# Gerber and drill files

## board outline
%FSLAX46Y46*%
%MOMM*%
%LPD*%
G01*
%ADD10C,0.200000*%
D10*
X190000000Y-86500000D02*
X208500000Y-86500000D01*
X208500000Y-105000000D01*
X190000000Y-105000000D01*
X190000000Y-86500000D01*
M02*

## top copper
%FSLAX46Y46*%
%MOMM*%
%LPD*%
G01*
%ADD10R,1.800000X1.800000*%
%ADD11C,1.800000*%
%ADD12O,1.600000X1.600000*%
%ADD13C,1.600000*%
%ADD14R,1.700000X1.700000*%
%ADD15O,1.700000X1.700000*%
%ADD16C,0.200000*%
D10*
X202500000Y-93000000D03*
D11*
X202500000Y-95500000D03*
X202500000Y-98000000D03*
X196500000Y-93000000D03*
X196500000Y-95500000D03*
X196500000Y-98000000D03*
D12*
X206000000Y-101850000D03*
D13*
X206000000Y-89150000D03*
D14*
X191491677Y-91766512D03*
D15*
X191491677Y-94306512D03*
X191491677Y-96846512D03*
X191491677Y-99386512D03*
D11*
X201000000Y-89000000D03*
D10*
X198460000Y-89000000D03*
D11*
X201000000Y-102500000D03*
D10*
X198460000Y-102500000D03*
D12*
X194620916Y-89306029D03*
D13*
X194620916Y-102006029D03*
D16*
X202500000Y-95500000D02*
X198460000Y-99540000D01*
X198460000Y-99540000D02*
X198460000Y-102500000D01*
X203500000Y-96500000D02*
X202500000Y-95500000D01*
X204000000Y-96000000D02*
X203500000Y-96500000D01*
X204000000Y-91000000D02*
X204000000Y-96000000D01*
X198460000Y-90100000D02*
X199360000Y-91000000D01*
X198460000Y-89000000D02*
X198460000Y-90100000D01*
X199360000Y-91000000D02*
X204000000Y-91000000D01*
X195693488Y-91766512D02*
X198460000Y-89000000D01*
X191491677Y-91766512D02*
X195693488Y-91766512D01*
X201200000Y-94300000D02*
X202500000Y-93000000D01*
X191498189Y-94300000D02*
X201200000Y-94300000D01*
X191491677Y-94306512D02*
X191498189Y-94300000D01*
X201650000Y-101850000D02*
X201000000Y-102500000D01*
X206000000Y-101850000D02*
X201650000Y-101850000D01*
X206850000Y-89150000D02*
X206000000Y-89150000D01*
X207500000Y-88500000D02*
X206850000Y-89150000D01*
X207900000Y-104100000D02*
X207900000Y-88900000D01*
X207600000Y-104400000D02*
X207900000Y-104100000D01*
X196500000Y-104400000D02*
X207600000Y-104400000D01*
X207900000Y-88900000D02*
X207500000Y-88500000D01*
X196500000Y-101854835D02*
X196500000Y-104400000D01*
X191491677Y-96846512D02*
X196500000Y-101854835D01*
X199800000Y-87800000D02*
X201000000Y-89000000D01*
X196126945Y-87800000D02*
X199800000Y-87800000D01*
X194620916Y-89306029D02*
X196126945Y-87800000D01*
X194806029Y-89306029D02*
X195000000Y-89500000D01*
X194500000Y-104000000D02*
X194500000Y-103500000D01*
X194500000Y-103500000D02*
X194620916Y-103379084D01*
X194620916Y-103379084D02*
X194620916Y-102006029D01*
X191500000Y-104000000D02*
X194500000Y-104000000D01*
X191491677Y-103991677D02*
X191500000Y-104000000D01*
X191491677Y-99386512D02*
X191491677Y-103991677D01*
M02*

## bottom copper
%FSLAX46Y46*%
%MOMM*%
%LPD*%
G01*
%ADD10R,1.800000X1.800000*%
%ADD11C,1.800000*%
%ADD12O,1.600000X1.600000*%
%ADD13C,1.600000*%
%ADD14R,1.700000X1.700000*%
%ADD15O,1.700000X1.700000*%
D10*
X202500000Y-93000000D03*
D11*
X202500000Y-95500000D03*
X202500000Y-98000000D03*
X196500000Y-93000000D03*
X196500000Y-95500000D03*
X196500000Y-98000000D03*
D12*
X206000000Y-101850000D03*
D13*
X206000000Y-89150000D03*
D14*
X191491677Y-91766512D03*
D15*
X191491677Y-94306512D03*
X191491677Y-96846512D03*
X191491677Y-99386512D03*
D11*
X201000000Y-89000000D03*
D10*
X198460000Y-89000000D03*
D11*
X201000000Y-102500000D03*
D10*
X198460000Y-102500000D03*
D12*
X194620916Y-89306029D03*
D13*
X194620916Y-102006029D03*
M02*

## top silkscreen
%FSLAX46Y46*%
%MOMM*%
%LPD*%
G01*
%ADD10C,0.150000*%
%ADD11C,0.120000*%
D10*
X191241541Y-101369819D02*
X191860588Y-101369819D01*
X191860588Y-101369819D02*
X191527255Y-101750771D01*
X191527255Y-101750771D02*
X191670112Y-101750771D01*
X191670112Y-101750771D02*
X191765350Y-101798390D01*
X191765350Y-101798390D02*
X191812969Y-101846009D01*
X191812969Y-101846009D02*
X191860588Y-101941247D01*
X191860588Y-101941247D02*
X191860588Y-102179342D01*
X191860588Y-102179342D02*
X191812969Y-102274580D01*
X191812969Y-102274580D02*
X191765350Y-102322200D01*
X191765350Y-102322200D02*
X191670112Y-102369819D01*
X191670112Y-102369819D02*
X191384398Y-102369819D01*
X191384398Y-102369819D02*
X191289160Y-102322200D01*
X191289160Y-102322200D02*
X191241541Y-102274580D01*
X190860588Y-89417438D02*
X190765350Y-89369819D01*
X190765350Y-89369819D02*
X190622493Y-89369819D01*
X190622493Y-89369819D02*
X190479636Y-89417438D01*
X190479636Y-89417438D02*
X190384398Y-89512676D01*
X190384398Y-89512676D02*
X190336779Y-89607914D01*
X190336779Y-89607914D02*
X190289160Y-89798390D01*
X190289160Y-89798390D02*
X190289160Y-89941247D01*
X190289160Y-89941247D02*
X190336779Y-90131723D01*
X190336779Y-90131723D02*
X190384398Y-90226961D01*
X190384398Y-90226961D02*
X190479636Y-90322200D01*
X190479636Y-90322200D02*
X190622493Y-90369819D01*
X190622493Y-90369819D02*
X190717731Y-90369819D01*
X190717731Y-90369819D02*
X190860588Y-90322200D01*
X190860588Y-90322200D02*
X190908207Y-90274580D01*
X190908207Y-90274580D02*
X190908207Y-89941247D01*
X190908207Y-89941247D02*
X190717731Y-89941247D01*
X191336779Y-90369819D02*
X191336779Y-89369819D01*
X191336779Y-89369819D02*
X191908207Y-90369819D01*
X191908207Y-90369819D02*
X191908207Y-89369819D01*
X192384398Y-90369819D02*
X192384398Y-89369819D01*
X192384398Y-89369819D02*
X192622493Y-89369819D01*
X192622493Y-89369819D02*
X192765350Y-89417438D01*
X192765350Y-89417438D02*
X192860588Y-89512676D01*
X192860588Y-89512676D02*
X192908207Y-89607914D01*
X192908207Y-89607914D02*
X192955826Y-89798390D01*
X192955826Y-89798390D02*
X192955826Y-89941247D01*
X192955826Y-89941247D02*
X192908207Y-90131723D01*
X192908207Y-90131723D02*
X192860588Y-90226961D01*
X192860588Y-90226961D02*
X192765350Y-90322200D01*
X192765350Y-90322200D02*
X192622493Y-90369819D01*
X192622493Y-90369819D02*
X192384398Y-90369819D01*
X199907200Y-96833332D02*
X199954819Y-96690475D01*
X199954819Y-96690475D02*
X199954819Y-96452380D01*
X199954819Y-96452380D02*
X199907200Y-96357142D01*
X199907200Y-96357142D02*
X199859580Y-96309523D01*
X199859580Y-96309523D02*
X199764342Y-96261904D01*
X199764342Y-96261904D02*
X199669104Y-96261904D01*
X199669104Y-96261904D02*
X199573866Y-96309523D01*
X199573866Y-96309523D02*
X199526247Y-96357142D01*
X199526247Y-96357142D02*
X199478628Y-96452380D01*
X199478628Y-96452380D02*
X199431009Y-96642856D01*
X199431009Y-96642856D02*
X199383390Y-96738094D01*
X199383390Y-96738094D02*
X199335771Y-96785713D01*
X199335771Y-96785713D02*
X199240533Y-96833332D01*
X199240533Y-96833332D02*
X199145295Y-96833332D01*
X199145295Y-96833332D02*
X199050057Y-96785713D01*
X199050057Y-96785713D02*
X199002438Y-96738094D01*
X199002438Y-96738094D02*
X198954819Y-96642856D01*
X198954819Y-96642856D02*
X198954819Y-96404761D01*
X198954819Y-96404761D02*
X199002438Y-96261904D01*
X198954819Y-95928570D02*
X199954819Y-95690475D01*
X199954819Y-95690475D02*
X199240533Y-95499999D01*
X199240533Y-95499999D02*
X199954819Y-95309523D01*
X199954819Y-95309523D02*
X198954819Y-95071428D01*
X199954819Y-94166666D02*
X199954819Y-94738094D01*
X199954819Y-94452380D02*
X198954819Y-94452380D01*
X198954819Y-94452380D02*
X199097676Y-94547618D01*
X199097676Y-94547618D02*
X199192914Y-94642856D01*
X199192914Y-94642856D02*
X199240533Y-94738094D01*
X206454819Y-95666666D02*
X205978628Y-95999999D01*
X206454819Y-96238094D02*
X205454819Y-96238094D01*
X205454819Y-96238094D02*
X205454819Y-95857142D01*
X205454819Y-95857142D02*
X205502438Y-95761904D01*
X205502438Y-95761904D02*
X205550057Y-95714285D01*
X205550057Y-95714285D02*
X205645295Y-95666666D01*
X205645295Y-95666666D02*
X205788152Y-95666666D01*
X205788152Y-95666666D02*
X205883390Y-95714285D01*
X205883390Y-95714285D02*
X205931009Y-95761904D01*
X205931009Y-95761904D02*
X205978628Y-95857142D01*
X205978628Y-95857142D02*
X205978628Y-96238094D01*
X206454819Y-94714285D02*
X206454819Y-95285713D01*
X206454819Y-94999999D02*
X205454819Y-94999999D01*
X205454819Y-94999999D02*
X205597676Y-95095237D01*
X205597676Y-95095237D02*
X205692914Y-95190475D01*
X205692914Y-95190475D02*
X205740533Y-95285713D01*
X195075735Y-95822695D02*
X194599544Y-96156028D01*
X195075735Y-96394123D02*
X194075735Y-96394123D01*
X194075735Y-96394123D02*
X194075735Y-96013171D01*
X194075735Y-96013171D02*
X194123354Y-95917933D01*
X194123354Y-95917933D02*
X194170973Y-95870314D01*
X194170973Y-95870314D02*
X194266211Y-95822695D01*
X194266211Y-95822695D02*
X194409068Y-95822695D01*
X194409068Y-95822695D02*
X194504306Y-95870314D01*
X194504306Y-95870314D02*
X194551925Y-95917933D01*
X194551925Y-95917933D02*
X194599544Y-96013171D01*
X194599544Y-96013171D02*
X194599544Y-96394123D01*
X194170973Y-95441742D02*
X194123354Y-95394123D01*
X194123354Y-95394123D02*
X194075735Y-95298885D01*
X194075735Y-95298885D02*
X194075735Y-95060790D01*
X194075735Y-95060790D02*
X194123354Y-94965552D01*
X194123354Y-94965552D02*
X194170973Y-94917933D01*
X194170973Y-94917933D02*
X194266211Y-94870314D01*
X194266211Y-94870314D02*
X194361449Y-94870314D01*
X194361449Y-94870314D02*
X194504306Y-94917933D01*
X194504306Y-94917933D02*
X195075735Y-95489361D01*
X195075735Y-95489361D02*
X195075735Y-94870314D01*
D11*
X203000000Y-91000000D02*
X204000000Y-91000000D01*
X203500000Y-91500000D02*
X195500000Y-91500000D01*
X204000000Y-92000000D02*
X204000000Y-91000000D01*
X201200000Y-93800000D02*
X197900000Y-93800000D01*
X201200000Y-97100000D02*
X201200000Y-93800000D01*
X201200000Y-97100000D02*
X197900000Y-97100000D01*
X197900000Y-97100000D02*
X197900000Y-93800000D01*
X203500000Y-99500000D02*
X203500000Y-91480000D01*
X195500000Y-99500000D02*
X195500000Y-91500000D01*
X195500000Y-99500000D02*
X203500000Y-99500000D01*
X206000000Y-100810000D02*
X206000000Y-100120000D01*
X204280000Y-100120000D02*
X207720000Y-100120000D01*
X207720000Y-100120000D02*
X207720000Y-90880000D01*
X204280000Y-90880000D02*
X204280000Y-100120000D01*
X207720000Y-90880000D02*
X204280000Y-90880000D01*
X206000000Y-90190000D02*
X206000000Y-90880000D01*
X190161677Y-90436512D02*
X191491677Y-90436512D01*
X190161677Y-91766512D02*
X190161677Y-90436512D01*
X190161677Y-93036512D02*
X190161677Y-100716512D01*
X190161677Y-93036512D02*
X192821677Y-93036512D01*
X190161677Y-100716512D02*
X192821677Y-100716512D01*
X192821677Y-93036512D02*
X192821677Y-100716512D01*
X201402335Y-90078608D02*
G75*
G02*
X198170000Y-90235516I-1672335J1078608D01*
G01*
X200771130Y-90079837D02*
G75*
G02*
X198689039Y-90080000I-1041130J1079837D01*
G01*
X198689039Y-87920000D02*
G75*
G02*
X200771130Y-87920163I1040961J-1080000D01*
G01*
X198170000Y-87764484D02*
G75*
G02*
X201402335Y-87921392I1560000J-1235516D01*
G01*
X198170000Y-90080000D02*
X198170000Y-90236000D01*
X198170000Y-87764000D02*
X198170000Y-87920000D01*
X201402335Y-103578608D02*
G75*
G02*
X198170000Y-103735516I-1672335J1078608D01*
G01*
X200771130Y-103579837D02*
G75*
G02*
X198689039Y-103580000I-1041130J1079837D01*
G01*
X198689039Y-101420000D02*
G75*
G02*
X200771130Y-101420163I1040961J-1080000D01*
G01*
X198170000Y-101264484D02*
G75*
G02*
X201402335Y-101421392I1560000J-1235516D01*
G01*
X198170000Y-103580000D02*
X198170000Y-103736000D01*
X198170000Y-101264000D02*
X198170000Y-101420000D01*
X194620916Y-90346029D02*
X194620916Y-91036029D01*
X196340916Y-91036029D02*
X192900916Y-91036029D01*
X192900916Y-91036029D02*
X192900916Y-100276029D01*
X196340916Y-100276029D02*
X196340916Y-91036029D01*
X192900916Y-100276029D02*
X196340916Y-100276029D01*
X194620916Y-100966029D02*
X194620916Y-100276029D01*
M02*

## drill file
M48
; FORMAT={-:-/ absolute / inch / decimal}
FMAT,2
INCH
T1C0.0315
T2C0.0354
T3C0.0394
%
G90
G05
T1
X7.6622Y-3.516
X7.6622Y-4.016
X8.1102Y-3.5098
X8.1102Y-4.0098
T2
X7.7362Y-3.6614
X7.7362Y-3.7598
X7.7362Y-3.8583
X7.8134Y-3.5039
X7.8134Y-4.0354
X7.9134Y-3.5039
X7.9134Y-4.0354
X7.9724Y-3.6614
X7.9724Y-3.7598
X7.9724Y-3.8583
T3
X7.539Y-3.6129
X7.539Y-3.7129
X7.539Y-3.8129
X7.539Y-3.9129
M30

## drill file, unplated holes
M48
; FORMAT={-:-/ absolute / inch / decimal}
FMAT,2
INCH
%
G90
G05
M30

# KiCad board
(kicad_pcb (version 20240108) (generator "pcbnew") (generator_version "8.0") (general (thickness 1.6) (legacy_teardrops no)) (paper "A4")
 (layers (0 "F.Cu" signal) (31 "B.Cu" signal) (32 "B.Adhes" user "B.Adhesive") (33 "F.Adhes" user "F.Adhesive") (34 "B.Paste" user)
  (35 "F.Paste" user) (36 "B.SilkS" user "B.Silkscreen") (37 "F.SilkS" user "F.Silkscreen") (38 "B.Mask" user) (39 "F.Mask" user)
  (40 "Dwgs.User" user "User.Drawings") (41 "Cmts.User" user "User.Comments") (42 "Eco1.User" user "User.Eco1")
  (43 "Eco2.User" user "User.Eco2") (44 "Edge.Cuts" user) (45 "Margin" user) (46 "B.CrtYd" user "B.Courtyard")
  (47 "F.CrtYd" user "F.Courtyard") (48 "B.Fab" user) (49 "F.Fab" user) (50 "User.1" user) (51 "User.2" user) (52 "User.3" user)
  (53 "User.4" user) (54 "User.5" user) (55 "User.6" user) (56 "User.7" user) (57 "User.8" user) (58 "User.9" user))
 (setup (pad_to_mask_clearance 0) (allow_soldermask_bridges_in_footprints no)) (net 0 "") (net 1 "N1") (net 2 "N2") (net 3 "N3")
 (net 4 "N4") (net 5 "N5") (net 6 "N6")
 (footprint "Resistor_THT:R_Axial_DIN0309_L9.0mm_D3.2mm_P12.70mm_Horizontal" (layer "F.Cu") (at 194.620916 102.006029 90)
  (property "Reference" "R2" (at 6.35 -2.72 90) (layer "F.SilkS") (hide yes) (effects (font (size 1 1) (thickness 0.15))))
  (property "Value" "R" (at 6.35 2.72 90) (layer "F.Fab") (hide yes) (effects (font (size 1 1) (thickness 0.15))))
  (fp_line (start 10.97 -1.72) (end 1.73 -1.72) (stroke (width 0.12) (type solid)) (layer "F.SilkS"))
  (fp_line (start 1.73 -1.72) (end 1.73 1.72) (stroke (width 0.12) (type solid)) (layer "F.SilkS"))
  (fp_line (start 11.66 0) (end 10.97 0) (stroke (width 0.12) (type solid)) (layer "F.SilkS"))
  (fp_line (start 1.04 0) (end 1.73 0) (stroke (width 0.12) (type solid)) (layer "F.SilkS"))
  (fp_line (start 10.97 1.72) (end 10.97 -1.72) (stroke (width 0.12) (type solid)) (layer "F.SilkS"))
  (fp_line (start 1.73 1.72) (end 10.97 1.72) (stroke (width 0.12) (type solid)) (layer "F.SilkS"))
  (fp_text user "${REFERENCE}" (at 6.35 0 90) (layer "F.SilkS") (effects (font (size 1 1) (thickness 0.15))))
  (pad "1" thru_hole circle (at 0 0 90) (size 1.6 1.6) (drill 0.8) (layers "*.Cu" "*.Mask") (remove_unused_layers no) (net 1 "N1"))
  (pad "2" thru_hole oval (at 12.7 0 90) (size 1.6 1.6) (drill 0.8) (layers "*.Cu" "*.Mask") (remove_unused_layers no) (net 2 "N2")))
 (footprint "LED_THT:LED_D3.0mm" (layer "F.Cu") (at 198.46 102.5)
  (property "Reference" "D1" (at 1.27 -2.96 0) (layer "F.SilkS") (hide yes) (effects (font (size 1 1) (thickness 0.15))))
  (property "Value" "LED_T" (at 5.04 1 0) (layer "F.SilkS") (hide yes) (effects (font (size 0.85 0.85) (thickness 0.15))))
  (fp_line (start -0.29 -1.236) (end -0.29 -1.08) (stroke (width 0.12) (type solid)) (layer "F.SilkS"))
  (fp_line (start -0.29 1.08) (end -0.29 1.236) (stroke (width 0.12) (type solid)) (layer "F.SilkS"))
  (fp_arc (start -0.29 -1.235516) (mid 1.366487 -1.987659) (end 2.942335 -1.078608) (stroke (width 0.12) (type solid)) (layer "F.SilkS"))
  (fp_arc (start 0.229039 -1.08) (mid 1.270117 -1.5) (end 2.31113 -1.079837) (stroke (width 0.12) (type solid)) (layer "F.SilkS"))
  (fp_arc (start 2.31113 1.079837) (mid 1.270117 1.5) (end 0.229039 1.08) (stroke (width 0.12) (type solid)) (layer "F.SilkS"))
  (fp_arc (start 2.942335 1.078608) (mid 1.366487 1.987659) (end -0.29 1.235516) (stroke (width 0.12) (type solid)) (layer "F.SilkS"))
  (pad "1" thru_hole rect (at 0 0) (size 1.8 1.8) (drill 0.9) (layers "*.Cu" "*.Mask") (remove_unused_layers no) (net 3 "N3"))
  (pad "2" thru_hole circle (at 2.54 0) (size 1.8 1.8) (drill 0.9) (layers "*.Cu" "*.Mask") (remove_unused_layers no) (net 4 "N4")))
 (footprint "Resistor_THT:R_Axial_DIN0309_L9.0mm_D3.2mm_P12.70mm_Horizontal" (layer "F.Cu") (at 206 89.15 -90)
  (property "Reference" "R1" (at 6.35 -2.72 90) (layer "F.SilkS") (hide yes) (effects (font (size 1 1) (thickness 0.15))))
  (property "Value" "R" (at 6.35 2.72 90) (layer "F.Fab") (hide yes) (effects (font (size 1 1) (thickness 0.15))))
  (fp_line (start 1.73 1.72) (end 10.97 1.72) (stroke (width 0.12) (type solid)) (layer "F.SilkS"))
  (fp_line (start 10.97 1.72) (end 10.97 -1.72) (stroke (width 0.12) (type solid)) (layer "F.SilkS"))
  (fp_line (start 1.04 0) (end 1.73 0) (stroke (width 0.12) (type solid)) (layer "F.SilkS"))
  (fp_line (start 11.66 0) (end 10.97 0) (stroke (width 0.12) (type solid)) (layer "F.SilkS"))
  (fp_line (start 1.73 -1.72) (end 1.73 1.72) (stroke (width 0.12) (type solid)) (layer "F.SilkS"))
  (fp_line (start 10.97 -1.72) (end 1.73 -1.72) (stroke (width 0.12) (type solid)) (layer "F.SilkS"))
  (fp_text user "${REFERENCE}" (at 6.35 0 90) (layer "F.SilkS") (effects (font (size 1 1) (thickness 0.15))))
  (pad "1" thru_hole circle (at 0 0 270) (size 1.6 1.6) (drill 0.8) (layers "*.Cu" "*.Mask") (remove_unused_layers no) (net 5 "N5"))
  (pad "2" thru_hole oval (at 12.7 0 270) (size 1.6 1.6) (drill 0.8) (layers "*.Cu" "*.Mask") (remove_unused_layers no) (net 4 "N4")))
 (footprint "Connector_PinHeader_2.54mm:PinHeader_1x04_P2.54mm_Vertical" (layer "F.Cu") (at 191.491677 91.766512)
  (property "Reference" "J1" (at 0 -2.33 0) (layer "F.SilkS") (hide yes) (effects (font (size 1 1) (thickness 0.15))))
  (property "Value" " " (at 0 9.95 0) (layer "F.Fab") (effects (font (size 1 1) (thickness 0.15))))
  (fp_line (start -1.33 -1.33) (end 0 -1.33) (stroke (width 0.12) (type solid)) (layer "F.SilkS"))
  (fp_line (start -1.33 0) (end -1.33 -1.33) (stroke (width 0.12) (type solid)) (layer "F.SilkS"))
  (fp_line (start -1.33 1.27) (end -1.33 8.95) (stroke (width 0.12) (type solid)) (layer "F.SilkS"))
  (fp_line (start -1.33 1.27) (end 1.33 1.27) (stroke (width 0.12) (type solid)) (layer "F.SilkS"))
  (fp_line (start -1.33 8.95) (end 1.33 8.95) (stroke (width 0.12) (type solid)) (layer "F.SilkS"))
  (fp_line (start 1.33 1.27) (end 1.33 8.95) (stroke (width 0.12) (type solid)) (layer "F.SilkS"))
  (pad "1" thru_hole rect (at 0 0) (size 1.7 1.7) (drill 1) (layers "*.Cu" "*.Mask") (remove_unused_layers no) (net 3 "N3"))
  (pad "2" thru_hole oval (at 0 2.54) (size 1.7 1.7) (drill 1) (layers "*.Cu" "*.Mask") (remove_unused_layers no) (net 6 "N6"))
  (pad "3" thru_hole oval (at 0 5.08) (size 1.7 1.7) (drill 1) (layers "*.Cu" "*.Mask") (remove_unused_layers no) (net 5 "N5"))
  (pad "4" thru_hole oval (at 0 7.62) (size 1.7 1.7) (drill 1) (layers "*.Cu" "*.Mask") (remove_unused_layers no) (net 1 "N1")))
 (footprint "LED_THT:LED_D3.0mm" (layer "F.Cu") (at 198.46 89)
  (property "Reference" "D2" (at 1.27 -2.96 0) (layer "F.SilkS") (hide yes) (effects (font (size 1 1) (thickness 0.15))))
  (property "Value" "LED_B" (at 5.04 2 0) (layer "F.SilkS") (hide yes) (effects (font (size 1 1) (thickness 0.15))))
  (fp_line (start -0.29 -1.236) (end -0.29 -1.08) (stroke (width 0.12) (type solid)) (layer "F.SilkS"))
  (fp_line (start -0.29 1.08) (end -0.29 1.236) (stroke (width 0.12) (type solid)) (layer "F.SilkS"))
  (fp_arc (start -0.29 -1.235516) (mid 1.366487 -1.987659) (end 2.942335 -1.078608) (stroke (width 0.12) (type solid)) (layer "F.SilkS"))
  (fp_arc (start 0.229039 -1.08) (mid 1.270117 -1.5) (end 2.31113 -1.079837) (stroke (width 0.12) (type solid)) (layer "F.SilkS"))
  (fp_arc (start 2.31113 1.079837) (mid 1.270117 1.5) (end 0.229039 1.08) (stroke (width 0.12) (type solid)) (layer "F.SilkS"))
  (fp_arc (start 2.942335 1.078608) (mid 1.366487 1.987659) (end -0.29 1.235516) (stroke (width 0.12) (type solid)) (layer "F.SilkS"))
  (pad "1" thru_hole rect (at 0 0) (size 1.8 1.8) (drill 0.9) (layers "*.Cu" "*.Mask") (remove_unused_layers no) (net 3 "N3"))
  (pad "2" thru_hole circle (at 2.54 0) (size 1.8 1.8) (drill 0.9) (layers "*.Cu" "*.Mask") (remove_unused_layers no) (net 2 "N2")))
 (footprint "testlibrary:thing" (layer "F.Cu") (at 194 90 -90)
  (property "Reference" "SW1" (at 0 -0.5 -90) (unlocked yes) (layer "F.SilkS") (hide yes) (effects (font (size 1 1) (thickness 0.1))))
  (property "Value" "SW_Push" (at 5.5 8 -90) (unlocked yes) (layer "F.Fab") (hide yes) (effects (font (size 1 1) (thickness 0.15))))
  (fp_line (start 9.5 -1.5) (end 1.5 -1.5) (stroke (width 0.12) (type solid)) (layer "F.SilkS"))
  (fp_line (start 9.5 -1.5) (end 9.5 -9.5) (stroke (width 0.12) (type solid)) (layer "F.SilkS"))
  (fp_line (start 7.1 -3.9) (end 3.8 -3.9) (stroke (width 0.12) (type solid)) (layer "F.SilkS"))
  (fp_line (start 3.8 -7.2) (end 3.8 -3.9) (stroke (width 0.12) (type solid)) (layer "F.SilkS"))
  (fp_line (start 7.1 -7.2) (end 7.1 -3.9) (stroke (width 0.12) (type solid)) (layer "F.SilkS"))
  (fp_line (start 7.1 -7.2) (end 3.8 -7.2) (stroke (width 0.12) (type solid)) (layer "F.SilkS"))
  (fp_line (start 1 -9) (end 1 -10) (stroke (width 0.12) (type solid)) (layer "F.SilkS"))
  (fp_line (start 1.5 -9.5) (end 1.5 -1.5) (stroke (width 0.12) (type solid)) (layer "F.SilkS"))
  (fp_line (start 9.5 -9.5) (end 1.48 -9.5) (stroke (width 0.12) (type solid)) (layer "F.SilkS"))
  (fp_line (start 2 -10) (end 1 -10) (stroke (width 0.12) (type solid)) (layer "F.SilkS"))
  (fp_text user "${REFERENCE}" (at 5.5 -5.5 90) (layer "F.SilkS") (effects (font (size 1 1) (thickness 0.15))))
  (pad "1" thru_hole rect (at 3 -8.5 270) (size 1.8 1.8) (drill 0.9) (layers "*.Cu" "*.Mask") (remove_unused_layers no) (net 6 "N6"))
  (pad "2" thru_hole circle (at 5.5 -8.5 270) (size 1.8 1.8) (drill 0.9) (layers "*.Cu" "*.Mask") (remove_unused_layers no) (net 3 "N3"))
  (pad "3" thru_hole circle (at 8 -8.5 270) (size 1.8 1.8) (drill 0.9) (layers "*.Cu" "*.Mask") (remove_unused_layers no))
  (pad "4" thru_hole circle (at 3 -2.5 270) (size 1.8 1.8) (drill 0.9) (layers "*.Cu" "*.Mask") (remove_unused_layers no))
  (pad "5" thru_hole circle (at 5.5 -2.5 270) (size 1.8 1.8) (drill 0.9) (layers "*.Cu" "*.Mask") (remove_unused_layers no))
  (pad "6" thru_hole circle (at 8 -2.5 270) (size 1.8 1.8) (drill 0.9) (layers "*.Cu" "*.Mask") (remove_unused_layers no)))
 (gr_rect (start 190 86.5) (end 208.5 105) (stroke (width 0.2) (type default)) (fill none) (layer "Edge.Cuts"))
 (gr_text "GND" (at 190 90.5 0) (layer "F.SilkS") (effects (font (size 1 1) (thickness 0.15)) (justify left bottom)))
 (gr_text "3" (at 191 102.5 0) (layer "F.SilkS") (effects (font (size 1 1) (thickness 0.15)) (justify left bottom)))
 (segment (start 195.693488 91.766512) (end 198.46 89) (width 0.2) (layer "F.Cu") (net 3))
 (segment (start 191.491677 91.766512) (end 195.693488 91.766512) (width 0.2) (layer "F.Cu") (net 3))
 (segment (start 199.36 91) (end 204 91) (width 0.2) (layer "F.Cu") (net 3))
 (segment (start 198.46 89) (end 198.46 90.1) (width 0.2) (layer "F.Cu") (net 3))
 (segment (start 204 96) (end 203.5 96.5) (width 0.2) (layer "F.Cu") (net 3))
 (segment (start 202.5 95.5) (end 198.46 99.54) (width 0.2) (layer "F.Cu") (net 3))
 (segment (start 204 91) (end 204 96) (width 0.2) (layer "F.Cu") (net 3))
 (segment (start 198.46 99.54) (end 198.46 102.5) (width 0.2) (layer "F.Cu") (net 3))
 (segment (start 198.46 90.1) (end 199.36 91) (width 0.2) (layer "F.Cu") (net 3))
 (segment (start 203.5 96.5) (end 202.5 95.5) (width 0.2) (layer "F.Cu") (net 3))
 (segment (start 206 101.85) (end 201.65 101.85) (width 0.2) (layer "F.Cu") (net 4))
 (segment (start 201.65 101.85) (end 201 102.5) (width 0.2) (layer "F.Cu") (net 4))
 (segment (start 194.620916 89.306029) (end 196.126945 87.8) (width 0.2) (layer "F.Cu") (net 2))
 (segment (start 199.8 87.8) (end 201 89) (width 0.2) (layer "F.Cu") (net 2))
 (segment (start 194.806029 89.306029) (end 195 89.5) (width 0.2) (layer "F.Cu") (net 2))
 (segment (start 196.126945 87.8) (end 199.8 87.8) (width 0.2) (layer "F.Cu") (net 2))
 (segment (start 194.5 104) (end 194.5 103.5) (width 0.2) (layer "F.Cu") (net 1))
 (segment (start 191.5 104) (end 194.5 104) (width 0.2) (layer "F.Cu") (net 1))
 (segment (start 194.5 103.5) (end 194.620916 103.379084) (width 0.2) (layer "F.Cu") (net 1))
 (segment (start 191.491677 99.386512) (end 191.491677 103.991677) (width 0.2) (layer "F.Cu") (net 1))
 (segment (start 191.491677 103.991677) (end 191.5 104) (width 0.2) (layer "F.Cu") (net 1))
 (segment (start 194.620916 103.379084) (end 194.620916 102.006029) (width 0.2) (layer "F.Cu") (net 1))
 (segment (start 207.9 88.9) (end 207.5 88.5) (width 0.2) (layer "F.Cu") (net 5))
 (segment (start 196.5 104.4) (end 207.6 104.4) (width 0.2) (layer "F.Cu") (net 5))
 (segment (start 206.85 89.15) (end 206 89.15) (width 0.2) (layer "F.Cu") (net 5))
 (segment (start 207.6 104.4) (end 207.9 104.1) (width 0.2) (layer "F.Cu") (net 5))
 (segment (start 207.5 88.5) (end 206.85 89.15) (width 0.2) (layer "F.Cu") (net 5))
 (segment (start 207.9 104.1) (end 207.9 88.9) (width 0.2) (layer "F.Cu") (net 5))
 (segment (start 191.491677 96.846512) (end 196.5 101.854835) (width 0.2) (layer "F.Cu") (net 5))
 (segment (start 196.5 101.854835) (end 196.5 104.4) (width 0.2) (layer "F.Cu") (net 5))
 (segment (start 191.491677 94.306512) (end 191.498189 94.3) (width 0.2) (layer "F.Cu") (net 6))
 (segment (start 201.2 94.3) (end 202.5 93) (width 0.2) (layer "F.Cu") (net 6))
 (segment (start 191.498189 94.3) (end 201.2 94.3) (width 0.2) (layer "F.Cu") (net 6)))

